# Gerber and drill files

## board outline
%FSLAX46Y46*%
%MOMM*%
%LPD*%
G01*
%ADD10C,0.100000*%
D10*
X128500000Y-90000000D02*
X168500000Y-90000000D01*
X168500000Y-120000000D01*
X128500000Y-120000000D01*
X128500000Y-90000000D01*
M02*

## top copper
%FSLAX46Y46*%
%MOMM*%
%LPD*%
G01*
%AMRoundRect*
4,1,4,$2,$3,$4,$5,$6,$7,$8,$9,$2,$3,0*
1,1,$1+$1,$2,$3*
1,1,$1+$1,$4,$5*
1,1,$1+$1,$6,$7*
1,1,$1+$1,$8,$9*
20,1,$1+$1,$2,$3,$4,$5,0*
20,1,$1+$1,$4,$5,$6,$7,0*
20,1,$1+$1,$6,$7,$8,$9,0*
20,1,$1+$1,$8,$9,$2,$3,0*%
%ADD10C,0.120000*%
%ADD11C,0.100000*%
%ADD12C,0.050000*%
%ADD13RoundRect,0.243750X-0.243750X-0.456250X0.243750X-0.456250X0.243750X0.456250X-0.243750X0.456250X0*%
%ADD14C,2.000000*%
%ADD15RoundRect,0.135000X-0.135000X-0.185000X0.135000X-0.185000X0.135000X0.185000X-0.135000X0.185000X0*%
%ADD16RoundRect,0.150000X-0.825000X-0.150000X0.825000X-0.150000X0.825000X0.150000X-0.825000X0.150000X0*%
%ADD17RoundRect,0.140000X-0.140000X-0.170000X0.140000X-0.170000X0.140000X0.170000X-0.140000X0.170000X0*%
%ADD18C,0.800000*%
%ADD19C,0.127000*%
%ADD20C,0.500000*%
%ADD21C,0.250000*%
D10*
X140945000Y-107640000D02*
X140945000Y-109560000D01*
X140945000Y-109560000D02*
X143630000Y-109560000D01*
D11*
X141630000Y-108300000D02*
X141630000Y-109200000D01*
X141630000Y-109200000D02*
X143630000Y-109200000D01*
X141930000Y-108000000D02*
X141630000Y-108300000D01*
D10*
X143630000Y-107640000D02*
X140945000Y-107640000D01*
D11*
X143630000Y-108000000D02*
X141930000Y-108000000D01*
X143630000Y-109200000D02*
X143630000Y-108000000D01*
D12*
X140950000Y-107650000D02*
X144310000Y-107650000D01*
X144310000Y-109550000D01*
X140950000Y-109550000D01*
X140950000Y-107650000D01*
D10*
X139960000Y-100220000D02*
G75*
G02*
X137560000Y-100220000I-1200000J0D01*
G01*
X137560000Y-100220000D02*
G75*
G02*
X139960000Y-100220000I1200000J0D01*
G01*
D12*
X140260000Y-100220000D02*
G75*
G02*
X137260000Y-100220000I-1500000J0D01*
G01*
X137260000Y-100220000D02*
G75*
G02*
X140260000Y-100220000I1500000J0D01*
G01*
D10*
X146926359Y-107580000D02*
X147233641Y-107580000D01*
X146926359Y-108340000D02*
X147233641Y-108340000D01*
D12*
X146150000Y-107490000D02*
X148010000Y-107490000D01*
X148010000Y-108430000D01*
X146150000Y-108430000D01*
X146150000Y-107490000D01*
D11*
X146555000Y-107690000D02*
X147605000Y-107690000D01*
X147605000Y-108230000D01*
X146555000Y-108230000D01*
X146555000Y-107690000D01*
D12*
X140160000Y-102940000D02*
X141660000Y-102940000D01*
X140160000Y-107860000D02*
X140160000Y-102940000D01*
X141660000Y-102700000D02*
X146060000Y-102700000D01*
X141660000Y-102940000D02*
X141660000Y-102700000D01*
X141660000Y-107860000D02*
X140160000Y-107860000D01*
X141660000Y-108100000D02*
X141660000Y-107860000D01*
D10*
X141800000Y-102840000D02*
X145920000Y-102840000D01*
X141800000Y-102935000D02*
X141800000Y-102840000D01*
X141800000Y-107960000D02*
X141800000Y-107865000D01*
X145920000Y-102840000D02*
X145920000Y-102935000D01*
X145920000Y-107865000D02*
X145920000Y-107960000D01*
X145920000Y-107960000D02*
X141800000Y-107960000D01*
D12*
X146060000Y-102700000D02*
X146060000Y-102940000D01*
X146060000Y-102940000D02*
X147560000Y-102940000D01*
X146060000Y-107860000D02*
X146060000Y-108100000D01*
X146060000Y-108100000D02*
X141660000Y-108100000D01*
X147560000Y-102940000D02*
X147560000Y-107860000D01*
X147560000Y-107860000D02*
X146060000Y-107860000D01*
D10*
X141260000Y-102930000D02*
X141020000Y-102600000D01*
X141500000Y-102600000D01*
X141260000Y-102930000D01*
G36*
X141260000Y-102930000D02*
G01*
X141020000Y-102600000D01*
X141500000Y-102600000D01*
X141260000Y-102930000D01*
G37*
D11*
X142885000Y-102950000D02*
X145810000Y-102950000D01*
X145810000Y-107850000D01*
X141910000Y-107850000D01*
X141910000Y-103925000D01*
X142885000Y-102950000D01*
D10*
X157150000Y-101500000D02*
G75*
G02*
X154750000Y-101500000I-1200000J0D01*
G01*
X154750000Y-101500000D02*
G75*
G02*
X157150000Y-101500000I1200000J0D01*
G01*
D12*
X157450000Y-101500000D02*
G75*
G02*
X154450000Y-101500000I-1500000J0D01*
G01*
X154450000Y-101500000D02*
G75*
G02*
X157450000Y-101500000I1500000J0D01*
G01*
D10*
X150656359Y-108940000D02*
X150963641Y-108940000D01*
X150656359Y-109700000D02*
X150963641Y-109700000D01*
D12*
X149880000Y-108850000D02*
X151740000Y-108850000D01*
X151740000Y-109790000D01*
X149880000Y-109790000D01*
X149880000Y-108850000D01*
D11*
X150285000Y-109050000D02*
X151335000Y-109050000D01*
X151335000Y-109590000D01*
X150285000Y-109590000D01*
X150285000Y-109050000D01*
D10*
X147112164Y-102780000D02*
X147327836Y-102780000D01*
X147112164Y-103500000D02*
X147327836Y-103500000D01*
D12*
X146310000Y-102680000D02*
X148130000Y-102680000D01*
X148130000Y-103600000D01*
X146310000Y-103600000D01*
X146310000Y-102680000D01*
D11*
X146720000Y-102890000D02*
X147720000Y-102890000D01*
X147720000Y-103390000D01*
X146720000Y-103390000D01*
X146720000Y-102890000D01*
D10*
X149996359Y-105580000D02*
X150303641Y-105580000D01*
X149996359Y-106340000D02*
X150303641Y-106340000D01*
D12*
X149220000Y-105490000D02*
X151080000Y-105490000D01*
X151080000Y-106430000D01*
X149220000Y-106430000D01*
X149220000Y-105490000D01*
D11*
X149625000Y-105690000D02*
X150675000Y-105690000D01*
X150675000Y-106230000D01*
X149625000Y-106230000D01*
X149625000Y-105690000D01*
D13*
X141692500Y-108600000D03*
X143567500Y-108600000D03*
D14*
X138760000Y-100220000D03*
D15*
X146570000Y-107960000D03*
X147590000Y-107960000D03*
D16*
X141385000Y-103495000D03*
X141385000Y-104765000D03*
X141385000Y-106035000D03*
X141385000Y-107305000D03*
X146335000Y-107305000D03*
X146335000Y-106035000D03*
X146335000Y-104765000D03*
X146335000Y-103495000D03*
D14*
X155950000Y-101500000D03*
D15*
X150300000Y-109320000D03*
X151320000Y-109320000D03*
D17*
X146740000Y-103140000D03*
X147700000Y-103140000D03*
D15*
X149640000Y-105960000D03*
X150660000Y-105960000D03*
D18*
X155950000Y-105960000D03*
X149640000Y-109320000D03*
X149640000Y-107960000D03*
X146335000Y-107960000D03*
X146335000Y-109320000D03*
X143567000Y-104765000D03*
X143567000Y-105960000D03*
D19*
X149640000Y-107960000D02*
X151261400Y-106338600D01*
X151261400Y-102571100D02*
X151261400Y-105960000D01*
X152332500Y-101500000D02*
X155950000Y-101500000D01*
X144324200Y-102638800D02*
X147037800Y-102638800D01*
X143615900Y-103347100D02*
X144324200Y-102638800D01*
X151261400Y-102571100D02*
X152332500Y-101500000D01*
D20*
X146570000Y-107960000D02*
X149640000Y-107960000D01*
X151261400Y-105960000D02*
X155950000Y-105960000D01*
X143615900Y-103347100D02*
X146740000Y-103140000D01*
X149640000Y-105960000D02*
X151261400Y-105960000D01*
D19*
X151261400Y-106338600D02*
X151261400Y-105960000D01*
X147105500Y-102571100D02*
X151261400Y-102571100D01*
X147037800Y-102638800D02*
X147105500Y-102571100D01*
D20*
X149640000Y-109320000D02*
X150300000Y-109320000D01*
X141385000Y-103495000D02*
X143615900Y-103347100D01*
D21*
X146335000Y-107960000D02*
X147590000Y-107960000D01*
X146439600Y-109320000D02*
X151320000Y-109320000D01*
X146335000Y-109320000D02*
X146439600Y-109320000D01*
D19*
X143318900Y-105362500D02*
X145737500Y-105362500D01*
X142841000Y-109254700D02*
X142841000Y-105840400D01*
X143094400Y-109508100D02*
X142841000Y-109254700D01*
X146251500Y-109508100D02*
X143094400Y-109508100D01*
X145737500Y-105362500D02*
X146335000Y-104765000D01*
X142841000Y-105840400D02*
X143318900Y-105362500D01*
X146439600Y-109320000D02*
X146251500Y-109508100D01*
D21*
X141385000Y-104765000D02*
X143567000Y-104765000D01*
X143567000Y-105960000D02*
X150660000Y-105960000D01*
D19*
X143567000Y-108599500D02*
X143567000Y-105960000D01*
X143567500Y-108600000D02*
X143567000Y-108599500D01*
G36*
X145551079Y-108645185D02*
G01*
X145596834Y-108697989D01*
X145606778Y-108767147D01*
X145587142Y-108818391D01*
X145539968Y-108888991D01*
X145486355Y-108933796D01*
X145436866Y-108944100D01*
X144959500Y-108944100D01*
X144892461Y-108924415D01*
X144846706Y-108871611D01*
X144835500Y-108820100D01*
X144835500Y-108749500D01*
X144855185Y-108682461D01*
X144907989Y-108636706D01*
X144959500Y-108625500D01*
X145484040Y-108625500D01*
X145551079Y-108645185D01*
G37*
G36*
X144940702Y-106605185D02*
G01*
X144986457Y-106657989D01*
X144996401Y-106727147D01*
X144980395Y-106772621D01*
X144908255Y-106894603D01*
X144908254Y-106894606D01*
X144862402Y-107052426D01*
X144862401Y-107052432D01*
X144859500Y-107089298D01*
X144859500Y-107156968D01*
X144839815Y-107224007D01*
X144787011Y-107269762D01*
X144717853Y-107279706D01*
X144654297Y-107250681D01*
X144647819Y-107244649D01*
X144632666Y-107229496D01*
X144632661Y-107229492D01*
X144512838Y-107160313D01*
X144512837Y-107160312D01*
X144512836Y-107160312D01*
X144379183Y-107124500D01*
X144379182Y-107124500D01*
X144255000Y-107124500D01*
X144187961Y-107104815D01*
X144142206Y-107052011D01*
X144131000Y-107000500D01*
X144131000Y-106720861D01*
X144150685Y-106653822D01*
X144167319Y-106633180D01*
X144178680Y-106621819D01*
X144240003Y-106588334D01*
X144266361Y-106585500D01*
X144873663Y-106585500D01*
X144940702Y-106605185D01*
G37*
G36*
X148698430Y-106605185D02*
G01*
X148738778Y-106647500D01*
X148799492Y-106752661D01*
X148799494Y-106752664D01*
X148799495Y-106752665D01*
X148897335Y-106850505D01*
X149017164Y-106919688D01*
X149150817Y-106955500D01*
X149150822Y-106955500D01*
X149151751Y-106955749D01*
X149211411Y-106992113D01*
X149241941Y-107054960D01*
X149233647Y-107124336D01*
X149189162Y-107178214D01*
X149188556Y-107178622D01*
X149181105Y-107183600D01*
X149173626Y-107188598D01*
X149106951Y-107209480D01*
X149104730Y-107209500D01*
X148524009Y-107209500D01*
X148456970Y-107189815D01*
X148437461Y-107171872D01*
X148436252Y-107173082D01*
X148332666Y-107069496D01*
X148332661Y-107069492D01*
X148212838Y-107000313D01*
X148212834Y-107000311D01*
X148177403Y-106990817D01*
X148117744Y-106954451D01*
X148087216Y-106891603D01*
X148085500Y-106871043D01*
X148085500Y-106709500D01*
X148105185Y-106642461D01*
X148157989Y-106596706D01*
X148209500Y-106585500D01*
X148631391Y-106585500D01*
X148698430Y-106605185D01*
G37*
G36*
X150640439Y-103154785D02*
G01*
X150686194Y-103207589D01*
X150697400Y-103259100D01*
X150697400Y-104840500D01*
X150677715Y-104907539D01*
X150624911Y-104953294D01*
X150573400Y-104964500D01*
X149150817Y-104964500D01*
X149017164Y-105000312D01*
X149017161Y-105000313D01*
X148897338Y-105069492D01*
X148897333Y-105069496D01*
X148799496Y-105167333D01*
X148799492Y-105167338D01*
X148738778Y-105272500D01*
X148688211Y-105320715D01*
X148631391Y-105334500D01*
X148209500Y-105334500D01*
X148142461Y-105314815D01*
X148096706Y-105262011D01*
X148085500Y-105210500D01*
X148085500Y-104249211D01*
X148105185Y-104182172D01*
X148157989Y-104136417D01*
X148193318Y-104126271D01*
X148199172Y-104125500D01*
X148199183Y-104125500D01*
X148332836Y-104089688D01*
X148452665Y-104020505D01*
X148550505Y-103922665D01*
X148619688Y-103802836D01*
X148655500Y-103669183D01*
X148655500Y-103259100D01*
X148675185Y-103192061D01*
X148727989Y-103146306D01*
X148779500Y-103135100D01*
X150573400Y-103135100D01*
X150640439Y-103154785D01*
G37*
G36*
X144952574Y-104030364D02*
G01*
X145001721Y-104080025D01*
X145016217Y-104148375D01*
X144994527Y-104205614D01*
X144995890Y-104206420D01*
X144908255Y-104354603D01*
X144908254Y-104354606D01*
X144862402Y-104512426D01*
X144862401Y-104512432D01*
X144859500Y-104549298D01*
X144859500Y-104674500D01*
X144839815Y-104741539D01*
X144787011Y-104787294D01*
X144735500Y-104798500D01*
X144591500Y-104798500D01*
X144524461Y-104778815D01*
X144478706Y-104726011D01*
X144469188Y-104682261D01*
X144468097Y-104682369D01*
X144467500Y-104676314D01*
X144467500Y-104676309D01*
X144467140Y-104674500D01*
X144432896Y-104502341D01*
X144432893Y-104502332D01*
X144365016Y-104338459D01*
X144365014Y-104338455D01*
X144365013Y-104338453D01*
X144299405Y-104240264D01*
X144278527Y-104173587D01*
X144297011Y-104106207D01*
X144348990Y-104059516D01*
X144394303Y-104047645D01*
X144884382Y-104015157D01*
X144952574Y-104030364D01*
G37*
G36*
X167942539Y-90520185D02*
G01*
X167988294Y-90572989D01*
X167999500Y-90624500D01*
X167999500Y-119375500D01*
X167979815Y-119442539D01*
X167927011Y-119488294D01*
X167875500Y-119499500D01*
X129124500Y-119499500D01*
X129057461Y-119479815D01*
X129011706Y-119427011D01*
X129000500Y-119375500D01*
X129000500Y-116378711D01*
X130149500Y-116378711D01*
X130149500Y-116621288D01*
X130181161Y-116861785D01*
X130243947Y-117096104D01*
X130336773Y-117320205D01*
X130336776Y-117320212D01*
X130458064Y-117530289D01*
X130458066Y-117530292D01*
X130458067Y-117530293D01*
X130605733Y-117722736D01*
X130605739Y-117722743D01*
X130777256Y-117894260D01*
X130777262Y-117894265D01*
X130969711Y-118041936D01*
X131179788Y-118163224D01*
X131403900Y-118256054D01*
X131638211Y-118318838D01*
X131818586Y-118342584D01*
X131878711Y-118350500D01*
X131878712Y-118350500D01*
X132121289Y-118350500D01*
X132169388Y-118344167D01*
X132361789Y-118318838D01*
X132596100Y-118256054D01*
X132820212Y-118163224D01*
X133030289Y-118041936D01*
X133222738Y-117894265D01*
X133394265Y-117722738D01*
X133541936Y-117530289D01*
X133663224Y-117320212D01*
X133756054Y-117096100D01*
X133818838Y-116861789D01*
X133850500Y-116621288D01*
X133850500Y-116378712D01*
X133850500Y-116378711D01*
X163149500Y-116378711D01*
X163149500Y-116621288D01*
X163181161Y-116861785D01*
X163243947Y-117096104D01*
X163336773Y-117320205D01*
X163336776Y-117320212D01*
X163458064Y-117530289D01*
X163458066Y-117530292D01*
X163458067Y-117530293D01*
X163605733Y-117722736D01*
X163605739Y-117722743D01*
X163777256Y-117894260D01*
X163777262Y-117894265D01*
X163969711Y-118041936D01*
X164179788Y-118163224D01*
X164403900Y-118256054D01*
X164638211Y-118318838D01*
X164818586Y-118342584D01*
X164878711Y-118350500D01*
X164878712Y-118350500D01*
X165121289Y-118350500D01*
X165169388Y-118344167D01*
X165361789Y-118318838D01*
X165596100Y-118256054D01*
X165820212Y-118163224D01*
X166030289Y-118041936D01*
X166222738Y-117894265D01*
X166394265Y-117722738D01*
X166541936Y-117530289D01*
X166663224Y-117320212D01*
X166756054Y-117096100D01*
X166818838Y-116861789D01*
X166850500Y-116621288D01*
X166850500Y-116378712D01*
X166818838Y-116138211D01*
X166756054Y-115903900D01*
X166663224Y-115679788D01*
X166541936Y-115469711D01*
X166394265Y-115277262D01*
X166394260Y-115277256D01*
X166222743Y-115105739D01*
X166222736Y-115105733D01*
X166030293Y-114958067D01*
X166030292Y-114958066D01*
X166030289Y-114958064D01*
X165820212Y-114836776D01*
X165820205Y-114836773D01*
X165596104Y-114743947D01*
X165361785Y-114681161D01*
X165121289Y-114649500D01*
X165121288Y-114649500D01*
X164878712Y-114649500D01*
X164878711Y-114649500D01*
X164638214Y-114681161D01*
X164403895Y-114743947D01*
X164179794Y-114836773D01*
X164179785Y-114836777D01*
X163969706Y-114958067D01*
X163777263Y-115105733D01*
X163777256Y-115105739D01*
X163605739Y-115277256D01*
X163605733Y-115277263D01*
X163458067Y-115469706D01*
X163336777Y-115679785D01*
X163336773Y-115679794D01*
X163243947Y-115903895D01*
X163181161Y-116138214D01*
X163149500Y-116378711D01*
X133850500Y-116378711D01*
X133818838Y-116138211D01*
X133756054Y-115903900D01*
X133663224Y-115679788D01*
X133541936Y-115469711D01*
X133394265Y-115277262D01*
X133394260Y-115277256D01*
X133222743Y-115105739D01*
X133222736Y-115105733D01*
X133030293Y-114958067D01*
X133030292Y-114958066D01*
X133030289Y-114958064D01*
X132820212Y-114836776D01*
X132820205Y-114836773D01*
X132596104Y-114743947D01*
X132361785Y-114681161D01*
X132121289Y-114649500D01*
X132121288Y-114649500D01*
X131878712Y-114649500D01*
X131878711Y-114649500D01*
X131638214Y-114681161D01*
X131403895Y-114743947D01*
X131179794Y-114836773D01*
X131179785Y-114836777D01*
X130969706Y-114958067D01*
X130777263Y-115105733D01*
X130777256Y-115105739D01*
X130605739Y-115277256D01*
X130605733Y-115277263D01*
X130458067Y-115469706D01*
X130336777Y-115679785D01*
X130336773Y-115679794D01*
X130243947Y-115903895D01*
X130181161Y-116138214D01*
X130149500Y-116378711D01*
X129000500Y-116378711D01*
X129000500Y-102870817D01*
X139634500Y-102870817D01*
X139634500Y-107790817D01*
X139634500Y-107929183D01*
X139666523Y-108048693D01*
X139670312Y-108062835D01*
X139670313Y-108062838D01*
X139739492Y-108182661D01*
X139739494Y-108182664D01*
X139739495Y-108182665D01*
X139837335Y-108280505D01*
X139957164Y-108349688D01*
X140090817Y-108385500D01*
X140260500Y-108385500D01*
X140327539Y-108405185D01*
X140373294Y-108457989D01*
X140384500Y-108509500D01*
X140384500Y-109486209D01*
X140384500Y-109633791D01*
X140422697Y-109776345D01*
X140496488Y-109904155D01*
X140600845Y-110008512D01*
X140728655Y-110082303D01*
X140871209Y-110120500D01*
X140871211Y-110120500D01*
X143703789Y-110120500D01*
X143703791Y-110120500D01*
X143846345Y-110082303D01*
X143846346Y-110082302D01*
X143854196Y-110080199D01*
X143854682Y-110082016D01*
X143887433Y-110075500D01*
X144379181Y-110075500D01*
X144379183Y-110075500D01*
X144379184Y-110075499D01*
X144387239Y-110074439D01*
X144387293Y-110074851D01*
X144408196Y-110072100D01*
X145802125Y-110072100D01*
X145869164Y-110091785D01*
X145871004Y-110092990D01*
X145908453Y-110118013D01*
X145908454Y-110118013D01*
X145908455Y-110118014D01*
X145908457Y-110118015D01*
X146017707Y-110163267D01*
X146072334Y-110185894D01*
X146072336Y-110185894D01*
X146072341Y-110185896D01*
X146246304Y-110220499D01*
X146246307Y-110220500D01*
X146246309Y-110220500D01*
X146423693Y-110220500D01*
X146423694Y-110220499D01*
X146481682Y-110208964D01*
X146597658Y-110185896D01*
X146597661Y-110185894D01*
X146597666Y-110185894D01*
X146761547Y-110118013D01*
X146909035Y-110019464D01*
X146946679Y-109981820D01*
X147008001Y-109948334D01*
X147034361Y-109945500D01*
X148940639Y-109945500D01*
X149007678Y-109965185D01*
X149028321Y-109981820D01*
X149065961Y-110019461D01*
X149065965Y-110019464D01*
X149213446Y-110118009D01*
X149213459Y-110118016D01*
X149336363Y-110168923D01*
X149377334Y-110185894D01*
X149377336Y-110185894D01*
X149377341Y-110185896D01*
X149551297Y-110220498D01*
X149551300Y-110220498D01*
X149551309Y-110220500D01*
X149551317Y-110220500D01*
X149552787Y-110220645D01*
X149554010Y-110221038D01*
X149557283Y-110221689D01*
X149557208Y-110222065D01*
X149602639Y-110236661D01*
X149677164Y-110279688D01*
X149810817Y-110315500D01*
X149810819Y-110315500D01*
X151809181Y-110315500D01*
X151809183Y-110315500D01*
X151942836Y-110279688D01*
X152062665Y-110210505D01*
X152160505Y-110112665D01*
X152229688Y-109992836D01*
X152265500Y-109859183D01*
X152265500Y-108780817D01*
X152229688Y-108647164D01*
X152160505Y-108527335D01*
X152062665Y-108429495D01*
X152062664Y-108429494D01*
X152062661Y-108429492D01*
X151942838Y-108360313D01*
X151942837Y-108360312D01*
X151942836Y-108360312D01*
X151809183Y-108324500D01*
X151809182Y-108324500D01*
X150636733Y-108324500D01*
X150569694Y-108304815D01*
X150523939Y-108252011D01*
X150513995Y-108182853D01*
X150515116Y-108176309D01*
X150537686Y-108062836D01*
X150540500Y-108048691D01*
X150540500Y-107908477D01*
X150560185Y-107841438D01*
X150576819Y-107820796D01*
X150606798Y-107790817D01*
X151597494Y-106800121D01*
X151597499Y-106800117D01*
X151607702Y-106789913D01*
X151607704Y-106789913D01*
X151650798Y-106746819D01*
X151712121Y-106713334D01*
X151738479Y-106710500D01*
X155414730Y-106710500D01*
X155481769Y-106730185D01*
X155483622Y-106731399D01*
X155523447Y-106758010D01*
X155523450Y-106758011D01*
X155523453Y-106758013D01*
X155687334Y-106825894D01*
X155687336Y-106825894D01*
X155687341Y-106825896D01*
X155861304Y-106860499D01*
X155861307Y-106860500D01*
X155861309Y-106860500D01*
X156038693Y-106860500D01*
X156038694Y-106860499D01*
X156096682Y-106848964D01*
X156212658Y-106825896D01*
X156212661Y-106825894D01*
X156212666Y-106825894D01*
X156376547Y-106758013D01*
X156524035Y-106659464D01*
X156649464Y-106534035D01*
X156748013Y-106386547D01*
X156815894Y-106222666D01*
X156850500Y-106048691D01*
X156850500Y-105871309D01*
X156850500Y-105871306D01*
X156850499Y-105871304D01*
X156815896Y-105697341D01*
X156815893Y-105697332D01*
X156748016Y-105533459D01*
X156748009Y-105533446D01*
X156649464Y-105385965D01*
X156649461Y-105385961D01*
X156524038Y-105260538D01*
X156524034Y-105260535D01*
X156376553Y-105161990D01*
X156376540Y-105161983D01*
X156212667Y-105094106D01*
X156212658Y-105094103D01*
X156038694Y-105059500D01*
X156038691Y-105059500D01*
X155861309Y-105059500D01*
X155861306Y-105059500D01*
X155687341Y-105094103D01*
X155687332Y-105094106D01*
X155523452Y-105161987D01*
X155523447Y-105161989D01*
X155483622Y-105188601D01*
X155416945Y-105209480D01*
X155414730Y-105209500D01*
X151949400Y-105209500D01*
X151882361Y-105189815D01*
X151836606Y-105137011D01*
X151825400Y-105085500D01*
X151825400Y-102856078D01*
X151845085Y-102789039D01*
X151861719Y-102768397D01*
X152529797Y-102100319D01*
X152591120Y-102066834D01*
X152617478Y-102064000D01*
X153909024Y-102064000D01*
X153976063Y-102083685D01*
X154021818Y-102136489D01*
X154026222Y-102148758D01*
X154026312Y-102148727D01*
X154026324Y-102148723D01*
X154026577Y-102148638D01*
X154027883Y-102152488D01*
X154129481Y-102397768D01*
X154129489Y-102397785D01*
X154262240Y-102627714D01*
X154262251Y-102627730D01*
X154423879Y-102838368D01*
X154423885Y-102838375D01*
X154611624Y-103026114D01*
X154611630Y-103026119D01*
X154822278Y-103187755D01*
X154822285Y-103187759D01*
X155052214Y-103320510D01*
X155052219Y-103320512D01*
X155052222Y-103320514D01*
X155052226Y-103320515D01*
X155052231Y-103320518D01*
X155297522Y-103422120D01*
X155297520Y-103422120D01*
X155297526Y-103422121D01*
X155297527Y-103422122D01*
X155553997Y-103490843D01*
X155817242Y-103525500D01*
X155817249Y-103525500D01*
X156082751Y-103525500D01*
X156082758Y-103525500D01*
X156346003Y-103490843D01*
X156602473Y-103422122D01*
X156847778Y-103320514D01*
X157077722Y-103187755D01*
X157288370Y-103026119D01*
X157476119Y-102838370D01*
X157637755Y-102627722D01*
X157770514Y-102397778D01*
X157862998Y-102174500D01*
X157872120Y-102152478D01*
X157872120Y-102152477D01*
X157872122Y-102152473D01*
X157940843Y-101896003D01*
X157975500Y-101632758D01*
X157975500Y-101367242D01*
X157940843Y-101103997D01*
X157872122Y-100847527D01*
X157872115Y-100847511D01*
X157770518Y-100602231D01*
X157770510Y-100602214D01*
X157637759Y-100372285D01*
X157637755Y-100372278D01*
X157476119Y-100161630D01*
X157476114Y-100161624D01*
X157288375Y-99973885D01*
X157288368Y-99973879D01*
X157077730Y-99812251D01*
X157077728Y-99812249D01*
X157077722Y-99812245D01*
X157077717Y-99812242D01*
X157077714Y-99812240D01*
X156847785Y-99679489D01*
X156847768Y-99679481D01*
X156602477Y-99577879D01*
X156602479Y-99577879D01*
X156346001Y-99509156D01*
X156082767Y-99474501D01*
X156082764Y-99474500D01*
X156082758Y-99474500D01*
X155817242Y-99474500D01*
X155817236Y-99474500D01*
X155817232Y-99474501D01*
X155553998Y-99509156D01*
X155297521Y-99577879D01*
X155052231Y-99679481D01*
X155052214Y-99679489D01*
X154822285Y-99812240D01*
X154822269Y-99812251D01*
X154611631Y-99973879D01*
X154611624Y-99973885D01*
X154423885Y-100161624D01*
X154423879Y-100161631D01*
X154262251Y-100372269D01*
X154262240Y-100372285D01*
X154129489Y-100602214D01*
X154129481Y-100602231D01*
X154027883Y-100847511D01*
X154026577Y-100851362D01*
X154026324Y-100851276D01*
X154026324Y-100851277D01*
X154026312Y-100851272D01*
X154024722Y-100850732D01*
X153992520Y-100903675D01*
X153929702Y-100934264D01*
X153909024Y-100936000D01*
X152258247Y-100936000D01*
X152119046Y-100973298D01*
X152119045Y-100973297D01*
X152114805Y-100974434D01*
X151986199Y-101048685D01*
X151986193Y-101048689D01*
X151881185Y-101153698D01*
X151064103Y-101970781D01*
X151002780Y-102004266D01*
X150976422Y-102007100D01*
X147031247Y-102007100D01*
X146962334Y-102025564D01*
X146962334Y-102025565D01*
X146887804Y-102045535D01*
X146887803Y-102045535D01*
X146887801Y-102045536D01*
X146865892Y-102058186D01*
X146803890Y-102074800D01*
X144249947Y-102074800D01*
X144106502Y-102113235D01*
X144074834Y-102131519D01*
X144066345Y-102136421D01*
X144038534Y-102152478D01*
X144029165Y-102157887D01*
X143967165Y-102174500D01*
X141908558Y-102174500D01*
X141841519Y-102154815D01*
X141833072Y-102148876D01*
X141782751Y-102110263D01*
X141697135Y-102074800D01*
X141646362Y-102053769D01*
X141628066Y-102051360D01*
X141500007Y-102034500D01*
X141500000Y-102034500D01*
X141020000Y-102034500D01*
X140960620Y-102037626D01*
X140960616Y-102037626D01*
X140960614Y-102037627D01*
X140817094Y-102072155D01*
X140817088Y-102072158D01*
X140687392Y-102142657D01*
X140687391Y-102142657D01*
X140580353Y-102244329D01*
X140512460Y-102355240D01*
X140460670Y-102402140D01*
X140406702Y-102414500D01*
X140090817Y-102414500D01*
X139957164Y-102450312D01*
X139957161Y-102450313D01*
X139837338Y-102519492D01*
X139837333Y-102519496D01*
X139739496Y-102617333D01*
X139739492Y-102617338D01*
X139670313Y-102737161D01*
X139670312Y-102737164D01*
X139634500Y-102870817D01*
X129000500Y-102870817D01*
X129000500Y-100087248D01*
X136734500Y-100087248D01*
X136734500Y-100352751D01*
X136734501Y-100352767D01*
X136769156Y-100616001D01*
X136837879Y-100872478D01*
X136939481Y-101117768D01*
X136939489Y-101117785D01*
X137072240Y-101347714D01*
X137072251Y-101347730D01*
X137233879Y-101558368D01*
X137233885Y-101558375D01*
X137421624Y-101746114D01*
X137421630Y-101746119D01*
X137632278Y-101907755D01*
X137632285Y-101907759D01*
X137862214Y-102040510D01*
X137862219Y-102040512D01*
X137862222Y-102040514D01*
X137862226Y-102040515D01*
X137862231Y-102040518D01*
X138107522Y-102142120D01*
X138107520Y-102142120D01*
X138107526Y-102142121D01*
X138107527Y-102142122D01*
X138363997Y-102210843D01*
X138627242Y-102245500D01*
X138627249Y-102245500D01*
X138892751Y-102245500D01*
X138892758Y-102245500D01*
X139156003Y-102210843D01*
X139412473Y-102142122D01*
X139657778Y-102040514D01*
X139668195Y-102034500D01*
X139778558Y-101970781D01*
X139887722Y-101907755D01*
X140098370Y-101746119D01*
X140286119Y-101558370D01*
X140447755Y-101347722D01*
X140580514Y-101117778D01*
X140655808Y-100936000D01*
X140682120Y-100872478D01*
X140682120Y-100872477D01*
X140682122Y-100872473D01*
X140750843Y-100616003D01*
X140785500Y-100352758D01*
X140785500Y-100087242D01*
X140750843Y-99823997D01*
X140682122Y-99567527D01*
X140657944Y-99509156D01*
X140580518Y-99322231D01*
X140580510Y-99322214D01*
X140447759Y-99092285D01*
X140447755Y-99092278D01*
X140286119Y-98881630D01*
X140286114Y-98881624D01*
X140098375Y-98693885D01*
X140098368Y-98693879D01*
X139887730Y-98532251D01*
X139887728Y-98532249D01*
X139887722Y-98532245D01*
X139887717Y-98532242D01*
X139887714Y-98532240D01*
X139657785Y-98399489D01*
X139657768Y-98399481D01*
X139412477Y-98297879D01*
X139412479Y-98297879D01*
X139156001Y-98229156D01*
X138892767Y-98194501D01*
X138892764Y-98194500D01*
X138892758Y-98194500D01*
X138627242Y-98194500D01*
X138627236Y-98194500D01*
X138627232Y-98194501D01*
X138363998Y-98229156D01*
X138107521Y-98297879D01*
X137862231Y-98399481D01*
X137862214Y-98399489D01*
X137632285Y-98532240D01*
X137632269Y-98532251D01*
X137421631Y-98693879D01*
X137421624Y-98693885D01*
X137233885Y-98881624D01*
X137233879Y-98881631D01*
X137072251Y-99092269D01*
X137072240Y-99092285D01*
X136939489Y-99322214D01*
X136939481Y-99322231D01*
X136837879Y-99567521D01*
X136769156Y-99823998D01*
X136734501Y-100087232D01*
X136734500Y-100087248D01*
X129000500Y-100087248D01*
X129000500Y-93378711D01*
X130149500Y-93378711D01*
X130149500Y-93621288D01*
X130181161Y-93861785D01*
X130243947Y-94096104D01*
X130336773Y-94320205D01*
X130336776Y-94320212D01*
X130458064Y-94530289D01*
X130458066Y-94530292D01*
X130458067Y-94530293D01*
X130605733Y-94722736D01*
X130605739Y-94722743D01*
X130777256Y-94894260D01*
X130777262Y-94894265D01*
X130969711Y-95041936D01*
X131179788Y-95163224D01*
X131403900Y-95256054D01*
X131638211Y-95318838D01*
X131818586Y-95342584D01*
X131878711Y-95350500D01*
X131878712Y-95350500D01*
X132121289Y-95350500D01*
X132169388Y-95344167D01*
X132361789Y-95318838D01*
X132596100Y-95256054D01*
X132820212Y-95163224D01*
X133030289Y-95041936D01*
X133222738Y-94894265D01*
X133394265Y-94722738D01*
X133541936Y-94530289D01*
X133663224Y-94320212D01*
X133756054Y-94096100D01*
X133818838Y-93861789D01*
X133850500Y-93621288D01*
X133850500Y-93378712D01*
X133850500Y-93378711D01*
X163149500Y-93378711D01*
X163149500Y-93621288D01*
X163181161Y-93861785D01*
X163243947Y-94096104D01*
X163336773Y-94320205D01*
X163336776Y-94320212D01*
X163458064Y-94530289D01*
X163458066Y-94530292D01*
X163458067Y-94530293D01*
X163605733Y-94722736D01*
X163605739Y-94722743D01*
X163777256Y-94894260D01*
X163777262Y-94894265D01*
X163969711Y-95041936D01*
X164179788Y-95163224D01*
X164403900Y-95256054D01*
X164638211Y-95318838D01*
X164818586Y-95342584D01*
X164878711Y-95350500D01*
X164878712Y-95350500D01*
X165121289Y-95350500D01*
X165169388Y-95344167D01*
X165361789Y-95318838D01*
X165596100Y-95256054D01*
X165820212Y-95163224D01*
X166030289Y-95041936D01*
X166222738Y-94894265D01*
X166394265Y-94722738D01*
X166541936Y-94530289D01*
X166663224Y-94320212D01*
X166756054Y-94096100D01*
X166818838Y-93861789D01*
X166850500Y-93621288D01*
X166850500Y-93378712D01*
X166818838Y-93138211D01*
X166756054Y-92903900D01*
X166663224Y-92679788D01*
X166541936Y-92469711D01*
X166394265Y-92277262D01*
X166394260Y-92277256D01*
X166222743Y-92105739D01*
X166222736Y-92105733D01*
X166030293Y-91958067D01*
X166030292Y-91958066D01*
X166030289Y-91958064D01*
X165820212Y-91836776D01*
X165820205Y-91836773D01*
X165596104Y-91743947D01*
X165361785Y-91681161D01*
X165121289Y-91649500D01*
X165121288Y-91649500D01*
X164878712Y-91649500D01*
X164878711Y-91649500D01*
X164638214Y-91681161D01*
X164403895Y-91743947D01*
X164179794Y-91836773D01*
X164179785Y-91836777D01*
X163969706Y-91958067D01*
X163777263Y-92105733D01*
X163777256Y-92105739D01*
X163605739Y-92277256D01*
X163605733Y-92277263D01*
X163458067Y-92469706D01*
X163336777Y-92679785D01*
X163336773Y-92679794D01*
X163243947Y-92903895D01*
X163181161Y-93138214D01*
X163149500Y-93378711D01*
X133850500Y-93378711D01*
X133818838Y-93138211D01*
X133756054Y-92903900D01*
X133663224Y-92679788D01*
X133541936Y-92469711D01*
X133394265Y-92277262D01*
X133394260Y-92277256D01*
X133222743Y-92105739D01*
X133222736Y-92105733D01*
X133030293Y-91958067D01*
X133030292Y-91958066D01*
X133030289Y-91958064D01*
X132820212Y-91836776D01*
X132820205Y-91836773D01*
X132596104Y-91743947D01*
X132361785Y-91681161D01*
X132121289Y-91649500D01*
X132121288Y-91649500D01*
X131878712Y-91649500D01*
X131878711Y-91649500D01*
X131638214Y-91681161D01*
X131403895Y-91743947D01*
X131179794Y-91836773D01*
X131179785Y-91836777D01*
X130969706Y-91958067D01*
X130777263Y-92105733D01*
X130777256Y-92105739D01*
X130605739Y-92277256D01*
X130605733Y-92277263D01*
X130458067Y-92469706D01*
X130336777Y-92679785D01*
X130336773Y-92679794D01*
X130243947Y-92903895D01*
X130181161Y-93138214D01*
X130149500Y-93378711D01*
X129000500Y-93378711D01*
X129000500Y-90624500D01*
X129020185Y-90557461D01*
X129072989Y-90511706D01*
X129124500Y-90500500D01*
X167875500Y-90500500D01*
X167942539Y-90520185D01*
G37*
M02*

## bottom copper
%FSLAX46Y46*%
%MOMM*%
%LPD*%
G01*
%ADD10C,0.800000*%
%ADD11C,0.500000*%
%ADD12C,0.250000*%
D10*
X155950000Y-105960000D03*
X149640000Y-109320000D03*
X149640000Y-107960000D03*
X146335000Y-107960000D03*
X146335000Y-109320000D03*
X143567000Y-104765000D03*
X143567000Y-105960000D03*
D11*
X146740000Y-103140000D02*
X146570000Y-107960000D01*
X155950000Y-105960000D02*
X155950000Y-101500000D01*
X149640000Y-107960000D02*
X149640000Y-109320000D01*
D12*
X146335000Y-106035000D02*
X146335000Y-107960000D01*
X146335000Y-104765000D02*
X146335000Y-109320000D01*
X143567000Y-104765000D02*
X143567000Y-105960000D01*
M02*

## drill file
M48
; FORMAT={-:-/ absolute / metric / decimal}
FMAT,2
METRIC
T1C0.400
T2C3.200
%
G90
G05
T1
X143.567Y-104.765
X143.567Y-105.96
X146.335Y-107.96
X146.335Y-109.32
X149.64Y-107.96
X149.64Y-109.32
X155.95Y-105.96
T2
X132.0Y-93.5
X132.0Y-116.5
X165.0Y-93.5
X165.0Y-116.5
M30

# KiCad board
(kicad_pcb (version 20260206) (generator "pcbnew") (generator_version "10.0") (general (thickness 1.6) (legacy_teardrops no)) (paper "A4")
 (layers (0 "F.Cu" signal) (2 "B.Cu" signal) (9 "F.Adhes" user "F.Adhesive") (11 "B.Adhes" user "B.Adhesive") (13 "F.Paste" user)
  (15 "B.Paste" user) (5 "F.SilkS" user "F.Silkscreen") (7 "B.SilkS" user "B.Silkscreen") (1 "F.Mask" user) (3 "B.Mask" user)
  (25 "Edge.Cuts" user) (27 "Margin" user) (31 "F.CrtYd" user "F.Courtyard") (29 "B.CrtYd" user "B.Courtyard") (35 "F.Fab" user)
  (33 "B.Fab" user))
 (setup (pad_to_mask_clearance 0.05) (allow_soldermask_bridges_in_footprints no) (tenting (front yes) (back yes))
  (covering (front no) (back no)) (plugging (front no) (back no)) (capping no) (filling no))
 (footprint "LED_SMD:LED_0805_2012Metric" (layer "F.Cu") (at 142.63 108.6)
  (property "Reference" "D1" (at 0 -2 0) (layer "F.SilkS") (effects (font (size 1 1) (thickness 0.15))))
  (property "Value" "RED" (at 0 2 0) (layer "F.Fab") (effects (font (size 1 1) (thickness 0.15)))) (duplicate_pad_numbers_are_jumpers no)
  (fp_line (start -1.685 -0.96) (end -1.685 0.96) (stroke (width 0.12) (type solid)) (layer "F.Cu"))
  (fp_line (start -1.685 0.96) (end 1 0.96) (stroke (width 0.12) (type solid)) (layer "F.Cu"))
  (fp_line (start -1 -0.3) (end -1 0.6) (stroke (width 0.1) (type solid)) (layer "F.Cu"))
  (fp_line (start -1 0.6) (end 1 0.6) (stroke (width 0.1) (type solid)) (layer "F.Cu"))
  (fp_line (start -0.7 -0.6) (end -1 -0.3) (stroke (width 0.1) (type solid)) (layer "F.Cu"))
  (fp_line (start 1 -0.96) (end -1.685 -0.96) (stroke (width 0.12) (type solid)) (layer "F.Cu"))
  (fp_line (start 1 -0.6) (end -0.7 -0.6) (stroke (width 0.1) (type solid)) (layer "F.Cu"))
  (fp_line (start 1 0.6) (end 1 -0.6) (stroke (width 0.1) (type solid)) (layer "F.Cu"))
  (fp_rect (start -1.68 -0.95) (end 1.68 0.95) (stroke (width 0.05) (type solid)) (fill no) (layer "F.Cu"))
  (pad "1" smd roundrect (at -0.9375 0) (size 0.975 1.4) (layers "F.Cu" "F.Mask" "F.Paste") (roundrect_rratio 0.25) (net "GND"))
  (pad "2" smd roundrect (at 0.9375 0) (size 0.975 1.4) (layers "F.Cu" "F.Mask" "F.Paste") (roundrect_rratio 0.25) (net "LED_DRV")))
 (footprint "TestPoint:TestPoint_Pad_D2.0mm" (layer "F.Cu") (at 138.76 100.22)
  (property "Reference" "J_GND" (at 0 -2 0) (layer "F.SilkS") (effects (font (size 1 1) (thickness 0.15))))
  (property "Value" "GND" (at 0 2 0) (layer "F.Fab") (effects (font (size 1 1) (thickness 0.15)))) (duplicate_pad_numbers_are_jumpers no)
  (fp_circle (center 0 0) (end 0 1.2) (stroke (width 0.12) (type solid)) (fill no) (layer "F.Cu"))
  (fp_circle (center 0 0) (end 1.5 0) (stroke (width 0.05) (type solid)) (fill no) (layer "F.Cu"))
  (pad "1" smd circle (at 0 0) (size 2 2) (layers "F.Cu" "F.Mask") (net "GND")))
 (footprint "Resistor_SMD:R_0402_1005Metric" (layer "F.Cu") (at 147.08 107.96)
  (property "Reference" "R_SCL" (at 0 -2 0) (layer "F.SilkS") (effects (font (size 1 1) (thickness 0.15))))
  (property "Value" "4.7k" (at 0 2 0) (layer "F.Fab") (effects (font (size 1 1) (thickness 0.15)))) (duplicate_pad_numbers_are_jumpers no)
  (fp_line (start -0.153641 -0.38) (end 0.153641 -0.38) (stroke (width 0.12) (type solid)) (layer "F.Cu"))
  (fp_line (start -0.153641 0.38) (end 0.153641 0.38) (stroke (width 0.12) (type solid)) (layer "F.Cu"))
  (fp_rect (start -0.93 -0.47) (end 0.93 0.47) (stroke (width 0.05) (type solid)) (fill no) (layer "F.Cu"))
  (fp_rect (start -0.525 -0.27) (end 0.525 0.27) (stroke (width 0.1) (type solid)) (fill no) (layer "F.Cu"))
  (pad "1" smd roundrect (at -0.51 0) (size 0.54 0.64) (layers "F.Cu" "F.Mask" "F.Paste") (roundrect_rratio 0.25) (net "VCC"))
  (pad "2" smd roundrect (at 0.51 0) (size 0.54 0.64) (layers "F.Cu" "F.Mask" "F.Paste") (roundrect_rratio 0.25) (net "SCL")))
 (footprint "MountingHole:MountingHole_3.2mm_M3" (layer "F.Cu") (at 165 93.5)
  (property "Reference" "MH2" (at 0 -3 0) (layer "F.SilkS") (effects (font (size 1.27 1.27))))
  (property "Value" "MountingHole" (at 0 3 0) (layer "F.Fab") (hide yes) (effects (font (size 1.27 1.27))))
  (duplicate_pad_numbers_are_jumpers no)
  (pad "" np_thru_hole circle (at 0 0) (size 3.2 3.2) (drill 3.2) (layers "*.Cu" "*.Mask")))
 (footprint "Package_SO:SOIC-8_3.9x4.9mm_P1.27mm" (layer "F.Cu") (at 143.86 105.4)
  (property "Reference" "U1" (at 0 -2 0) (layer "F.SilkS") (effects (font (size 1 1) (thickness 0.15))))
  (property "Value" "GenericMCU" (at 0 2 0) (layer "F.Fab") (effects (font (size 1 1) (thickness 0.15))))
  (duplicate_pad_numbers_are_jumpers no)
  (fp_line (start -3.7 -2.46) (end -2.2 -2.46) (stroke (width 0.05) (type solid)) (layer "F.Cu"))
  (fp_line (start -3.7 2.46) (end -3.7 -2.46) (stroke (width 0.05) (type solid)) (layer "F.Cu"))
  (fp_line (start -2.2 -2.7) (end 2.2 -2.7) (stroke (width 0.05) (type solid)) (layer "F.Cu"))
  (fp_line (start -2.2 -2.46) (end -2.2 -2.7) (stroke (width 0.05) (type solid)) (layer "F.Cu"))
  (fp_line (start -2.2 2.46) (end -3.7 2.46) (stroke (width 0.05) (type solid)) (layer "F.Cu"))
  (fp_line (start -2.2 2.7) (end -2.2 2.46) (stroke (width 0.05) (type solid)) (layer "F.Cu"))
  (fp_line (start -2.06 -2.56) (end 2.06 -2.56) (stroke (width 0.12) (type solid)) (layer "F.Cu"))
  (fp_line (start -2.06 -2.465) (end -2.06 -2.56) (stroke (width 0.12) (type solid)) (layer "F.Cu"))
  (fp_line (start -2.06 2.56) (end -2.06 2.465) (stroke (width 0.12) (type solid)) (layer "F.Cu"))
  (fp_line (start 2.06 -2.56) (end 2.06 -2.465) (stroke (width 0.12) (type solid)) (layer "F.Cu"))
  (fp_line (start 2.06 2.465) (end 2.06 2.56) (stroke (width 0.12) (type solid)) (layer "F.Cu"))
  (fp_line (start 2.06 2.56) (end -2.06 2.56) (stroke (width 0.12) (type solid)) (layer "F.Cu"))
  (fp_line (start 2.2 -2.7) (end 2.2 -2.46) (stroke (width 0.05) (type solid)) (layer "F.Cu"))
  (fp_line (start 2.2 -2.46) (end 3.7 -2.46) (stroke (width 0.05) (type solid)) (layer "F.Cu"))
  (fp_line (start 2.2 2.46) (end 2.2 2.7) (stroke (width 0.05) (type solid)) (layer "F.Cu"))
  (fp_line (start 2.2 2.7) (end -2.2 2.7) (stroke (width 0.05) (type solid)) (layer "F.Cu"))
  (fp_line (start 3.7 -2.46) (end 3.7 2.46) (stroke (width 0.05) (type solid)) (layer "F.Cu"))
  (fp_line (start 3.7 2.46) (end 2.2 2.46) (stroke (width 0.05) (type solid)) (layer "F.Cu"))
  (fp_poly (pts (xy -2.6 -2.47) (xy -2.84 -2.8) (xy -2.36 -2.8)) (stroke (width 0.12) (type solid)) (fill yes) (layer "F.Cu"))
  (fp_poly
   (pts (xy -0.975 -2.45) (xy 1.95 -2.45) (xy 1.95 2.45) (xy -1.95 2.45) (xy -1.95 -1.475)) (stroke (width 0.1) (type solid)) (fill no)
   (layer "F.Cu"))
  (pad "1" smd roundrect (at -2.475 -1.905) (size 1.95 0.6) (layers "F.Cu" "F.Mask" "F.Paste") (roundrect_rratio 0.25) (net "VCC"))
  (pad "2" smd roundrect (at -2.475 -0.635) (size 1.95 0.6) (layers "F.Cu" "F.Mask" "F.Paste") (roundrect_rratio 0.25) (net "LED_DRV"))
  (pad "3" smd roundrect (at -2.475 0.635) (size 1.95 0.6) (layers "F.Cu" "F.Mask" "F.Paste") (roundrect_rratio 0.25) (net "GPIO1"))
  (pad "4" smd roundrect (at -2.475 1.905) (size 1.95 0.6) (layers "F.Cu" "F.Mask" "F.Paste") (roundrect_rratio 0.25) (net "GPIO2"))
  (pad "5" smd roundrect (at 2.475 1.905) (size 1.95 0.6) (layers "F.Cu" "F.Mask" "F.Paste") (roundrect_rratio 0.25) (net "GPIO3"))
  (pad "6" smd roundrect (at 2.475 0.635) (size 1.95 0.6) (layers "F.Cu" "F.Mask" "F.Paste") (roundrect_rratio 0.25) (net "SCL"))
  (pad "7" smd roundrect (at 2.475 -0.635) (size 1.95 0.6) (layers "F.Cu" "F.Mask" "F.Paste") (roundrect_rratio 0.25) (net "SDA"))
  (pad "8" smd roundrect (at 2.475 -1.905) (size 1.95 0.6) (layers "F.Cu" "F.Mask" "F.Paste") (roundrect_rratio 0.25) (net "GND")))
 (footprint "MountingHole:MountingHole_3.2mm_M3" (layer "F.Cu") (at 132 93.5)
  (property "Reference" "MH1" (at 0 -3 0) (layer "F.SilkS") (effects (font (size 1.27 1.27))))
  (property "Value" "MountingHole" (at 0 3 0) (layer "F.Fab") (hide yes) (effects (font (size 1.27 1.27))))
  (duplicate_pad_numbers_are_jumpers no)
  (pad "" np_thru_hole circle (at 0 0) (size 3.2 3.2) (drill 3.2) (layers "*.Cu" "*.Mask")))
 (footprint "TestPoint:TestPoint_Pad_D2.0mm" (layer "F.Cu") (at 155.95 101.5)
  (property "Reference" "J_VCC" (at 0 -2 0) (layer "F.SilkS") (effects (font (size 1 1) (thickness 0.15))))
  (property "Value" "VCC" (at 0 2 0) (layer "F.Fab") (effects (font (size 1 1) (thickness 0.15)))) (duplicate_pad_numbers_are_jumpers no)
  (fp_circle (center 0 0) (end 0 1.2) (stroke (width 0.12) (type solid)) (fill no) (layer "F.Cu"))
  (fp_circle (center 0 0) (end 1.5 0) (stroke (width 0.05) (type solid)) (fill no) (layer "F.Cu"))
  (pad "1" smd circle (at 0 0) (size 2 2) (layers "F.Cu" "F.Mask") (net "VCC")))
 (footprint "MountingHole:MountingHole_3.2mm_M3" (layer "F.Cu") (at 165 116.5)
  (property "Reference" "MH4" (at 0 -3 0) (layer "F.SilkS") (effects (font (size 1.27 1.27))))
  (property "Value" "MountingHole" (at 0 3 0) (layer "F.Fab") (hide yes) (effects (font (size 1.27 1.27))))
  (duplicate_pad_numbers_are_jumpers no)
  (pad "" np_thru_hole circle (at 0 0) (size 3.2 3.2) (drill 3.2) (layers "*.Cu" "*.Mask")))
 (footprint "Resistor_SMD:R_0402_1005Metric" (layer "F.Cu") (at 150.81 109.32)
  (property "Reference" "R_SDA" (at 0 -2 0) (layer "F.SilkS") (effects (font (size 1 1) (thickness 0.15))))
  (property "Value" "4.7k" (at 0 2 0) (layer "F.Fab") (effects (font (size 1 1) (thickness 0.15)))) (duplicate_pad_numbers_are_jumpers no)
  (fp_line (start -0.153641 -0.38) (end 0.153641 -0.38) (stroke (width 0.12) (type solid)) (layer "F.Cu"))
  (fp_line (start -0.153641 0.38) (end 0.153641 0.38) (stroke (width 0.12) (type solid)) (layer "F.Cu"))
  (fp_rect (start -0.93 -0.47) (end 0.93 0.47) (stroke (width 0.05) (type solid)) (fill no) (layer "F.Cu"))
  (fp_rect (start -0.525 -0.27) (end 0.525 0.27) (stroke (width 0.1) (type solid)) (fill no) (layer "F.Cu"))
  (pad "1" smd roundrect (at -0.51 0) (size 0.54 0.64) (layers "F.Cu" "F.Mask" "F.Paste") (roundrect_rratio 0.25) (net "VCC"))
  (pad "2" smd roundrect (at 0.51 0) (size 0.54 0.64) (layers "F.Cu" "F.Mask" "F.Paste") (roundrect_rratio 0.25) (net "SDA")))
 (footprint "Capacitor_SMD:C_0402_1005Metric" (layer "F.Cu") (at 147.22 103.14)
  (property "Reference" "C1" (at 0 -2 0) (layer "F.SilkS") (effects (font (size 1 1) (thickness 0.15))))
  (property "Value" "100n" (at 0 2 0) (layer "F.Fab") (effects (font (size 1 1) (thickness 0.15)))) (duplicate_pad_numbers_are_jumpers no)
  (fp_line (start -0.107836 -0.36) (end 0.107836 -0.36) (stroke (width 0.12) (type solid)) (layer "F.Cu"))
  (fp_line (start -0.107836 0.36) (end 0.107836 0.36) (stroke (width 0.12) (type solid)) (layer "F.Cu"))
  (fp_rect (start -0.91 -0.46) (end 0.91 0.46) (stroke (width 0.05) (type solid)) (fill no) (layer "F.Cu"))
  (fp_rect (start -0.5 -0.25) (end 0.5 0.25) (stroke (width 0.1) (type solid)) (fill no) (layer "F.Cu"))
  (pad "1" smd roundrect (at -0.48 0) (size 0.56 0.62) (layers "F.Cu" "F.Mask" "F.Paste") (roundrect_rratio 0.25) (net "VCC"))
  (pad "2" smd roundrect (at 0.48 0) (size 0.56 0.62) (layers "F.Cu" "F.Mask" "F.Paste") (roundrect_rratio 0.25) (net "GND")))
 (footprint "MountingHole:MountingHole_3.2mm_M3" (layer "F.Cu") (at 132 116.5)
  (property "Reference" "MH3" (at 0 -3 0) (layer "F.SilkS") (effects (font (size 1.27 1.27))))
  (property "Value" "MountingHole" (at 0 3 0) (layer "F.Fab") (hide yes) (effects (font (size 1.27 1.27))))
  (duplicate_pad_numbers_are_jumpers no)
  (pad "" np_thru_hole circle (at 0 0) (size 3.2 3.2) (drill 3.2) (layers "*.Cu" "*.Mask")))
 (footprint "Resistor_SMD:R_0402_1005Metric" (layer "F.Cu") (at 150.15 105.96)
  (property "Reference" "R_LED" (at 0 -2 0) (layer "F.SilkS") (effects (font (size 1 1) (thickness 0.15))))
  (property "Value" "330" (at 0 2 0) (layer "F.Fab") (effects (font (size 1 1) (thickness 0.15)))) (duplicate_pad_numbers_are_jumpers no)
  (fp_line (start -0.153641 -0.38) (end 0.153641 -0.38) (stroke (width 0.12) (type solid)) (layer "F.Cu"))
  (fp_line (start -0.153641 0.38) (end 0.153641 0.38) (stroke (width 0.12) (type solid)) (layer "F.Cu"))
  (fp_rect (start -0.93 -0.47) (end 0.93 0.47) (stroke (width 0.05) (type solid)) (fill no) (layer "F.Cu"))
  (fp_rect (start -0.525 -0.27) (end 0.525 0.27) (stroke (width 0.1) (type solid)) (fill no) (layer "F.Cu"))
  (pad "1" smd roundrect (at -0.51 0) (size 0.54 0.64) (layers "F.Cu" "F.Mask" "F.Paste") (roundrect_rratio 0.25) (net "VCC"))
  (pad "2" smd roundrect (at 0.51 0) (size 0.54 0.64) (layers "F.Cu" "F.Mask" "F.Paste") (roundrect_rratio 0.25) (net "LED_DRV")))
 (gr_rect (start 128.5 90) (end 168.5 120) (stroke (width 0.1) (type default)) (fill no) (layer "Edge.Cuts"))
 (segment (start 149.64 107.96) (end 151.2614 106.3386) (width 0.127) (layer "F.Cu") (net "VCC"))
 (segment (start 151.2614 102.5711) (end 151.2614 105.96) (width 0.127) (layer "F.Cu") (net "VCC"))
 (segment (start 152.3325 101.5) (end 155.95 101.5) (width 0.127) (layer "F.Cu") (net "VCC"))
 (segment (start 144.3242 102.6388) (end 147.0378 102.6388) (width 0.127) (layer "F.Cu") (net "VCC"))
 (segment (start 143.6159 103.3471) (end 144.3242 102.6388) (width 0.127) (layer "F.Cu") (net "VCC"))
 (segment (start 151.2614 102.5711) (end 152.3325 101.5) (width 0.127) (layer "F.Cu") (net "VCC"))
 (segment (start 146.57 107.96) (end 149.64 107.96) (width 0.5) (layer "F.Cu") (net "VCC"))
 (segment (start 151.2614 105.96) (end 155.95 105.96) (width 0.5) (layer "F.Cu") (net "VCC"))
 (segment (start 143.6159 103.3471) (end 146.74 103.14) (width 0.5) (layer "F.Cu") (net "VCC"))
 (segment (start 149.64 105.96) (end 151.2614 105.96) (width 0.5) (layer "F.Cu") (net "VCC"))
 (segment (start 151.2614 106.3386) (end 151.2614 105.96) (width 0.127) (layer "F.Cu") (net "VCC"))
 (segment (start 147.1055 102.5711) (end 151.2614 102.5711) (width 0.127) (layer "F.Cu") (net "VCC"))
 (segment (start 147.0378 102.6388) (end 147.1055 102.5711) (width 0.127) (layer "F.Cu") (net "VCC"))
 (segment (start 149.64 109.32) (end 150.3 109.32) (width 0.5) (layer "F.Cu") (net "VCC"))
 (segment (start 141.385 103.495) (end 143.6159 103.3471) (width 0.5) (layer "F.Cu") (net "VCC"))
 (via (at 155.95 105.96) (size 0.8) (drill 0.4) (layers "F.Cu" "B.Cu") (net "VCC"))
 (via (at 149.64 109.32) (size 0.8) (drill 0.4) (layers "F.Cu" "B.Cu") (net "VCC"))
 (via (at 149.64 107.96) (size 0.8) (drill 0.4) (layers "F.Cu" "B.Cu") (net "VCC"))
 (segment (start 146.74 103.14) (end 146.57 107.96) (width 0.5) (layer "B.Cu") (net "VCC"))
 (segment (start 155.95 105.96) (end 155.95 101.5) (width 0.5) (layer "B.Cu") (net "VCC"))
 (segment (start 149.64 107.96) (end 149.64 109.32) (width 0.5) (layer "B.Cu") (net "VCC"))
 (segment (start 146.335 107.96) (end 147.59 107.96) (width 0.25) (layer "F.Cu") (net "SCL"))
 (via (at 146.335 107.96) (size 0.8) (drill 0.4) (layers "F.Cu" "B.Cu") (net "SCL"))
 (segment (start 146.335 106.035) (end 146.335 107.96) (width 0.25) (layer "B.Cu") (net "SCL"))
 (segment (start 146.4396 109.32) (end 151.32 109.32) (width 0.25) (layer "F.Cu") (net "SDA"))
 (segment (start 146.335 109.32) (end 146.4396 109.32) (width 0.25) (layer "F.Cu") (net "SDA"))
 (segment (start 143.3189 105.3625) (end 145.7375 105.3625) (width 0.127) (layer "F.Cu") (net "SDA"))
 (segment (start 142.841 109.2547) (end 142.841 105.8404) (width 0.127) (layer "F.Cu") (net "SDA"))
 (segment (start 143.0944 109.5081) (end 142.841 109.2547) (width 0.127) (layer "F.Cu") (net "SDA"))
 (segment (start 146.2515 109.5081) (end 143.0944 109.5081) (width 0.127) (layer "F.Cu") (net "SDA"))
 (segment (start 145.7375 105.3625) (end 146.335 104.765) (width 0.127) (layer "F.Cu") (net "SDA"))
 (segment (start 142.841 105.8404) (end 143.3189 105.3625) (width 0.127) (layer "F.Cu") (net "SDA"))
 (segment (start 146.4396 109.32) (end 146.2515 109.5081) (width 0.127) (layer "F.Cu") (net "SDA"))
 (via (at 146.335 109.32) (size 0.8) (drill 0.4) (layers "F.Cu" "B.Cu") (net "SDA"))
 (segment (start 146.335 104.765) (end 146.335 109.32) (width 0.25) (layer "B.Cu") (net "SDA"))
 (segment (start 141.385 104.765) (end 143.567 104.765) (width 0.25) (layer "F.Cu") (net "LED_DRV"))
 (segment (start 143.567 105.96) (end 150.66 105.96) (width 0.25) (layer "F.Cu") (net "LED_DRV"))
 (segment (start 143.567 108.5995) (end 143.567 105.96) (width 0.127) (layer "F.Cu") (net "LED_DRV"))
 (segment (start 143.5675 108.6) (end 143.567 108.5995) (width 0.127) (layer "F.Cu") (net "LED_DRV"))
 (via (at 143.567 104.765) (size 0.8) (drill 0.4) (layers "F.Cu" "B.Cu") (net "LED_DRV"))
 (via (at 143.567 105.96) (size 0.8) (drill 0.4) (layers "F.Cu" "B.Cu") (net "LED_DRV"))
 (segment (start 143.567 104.765) (end 143.567 105.96) (width 0.25) (layer "B.Cu") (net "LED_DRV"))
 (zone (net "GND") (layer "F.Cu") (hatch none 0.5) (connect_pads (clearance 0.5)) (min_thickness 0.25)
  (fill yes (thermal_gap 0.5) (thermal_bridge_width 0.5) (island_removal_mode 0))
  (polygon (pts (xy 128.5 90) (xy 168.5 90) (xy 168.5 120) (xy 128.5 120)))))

